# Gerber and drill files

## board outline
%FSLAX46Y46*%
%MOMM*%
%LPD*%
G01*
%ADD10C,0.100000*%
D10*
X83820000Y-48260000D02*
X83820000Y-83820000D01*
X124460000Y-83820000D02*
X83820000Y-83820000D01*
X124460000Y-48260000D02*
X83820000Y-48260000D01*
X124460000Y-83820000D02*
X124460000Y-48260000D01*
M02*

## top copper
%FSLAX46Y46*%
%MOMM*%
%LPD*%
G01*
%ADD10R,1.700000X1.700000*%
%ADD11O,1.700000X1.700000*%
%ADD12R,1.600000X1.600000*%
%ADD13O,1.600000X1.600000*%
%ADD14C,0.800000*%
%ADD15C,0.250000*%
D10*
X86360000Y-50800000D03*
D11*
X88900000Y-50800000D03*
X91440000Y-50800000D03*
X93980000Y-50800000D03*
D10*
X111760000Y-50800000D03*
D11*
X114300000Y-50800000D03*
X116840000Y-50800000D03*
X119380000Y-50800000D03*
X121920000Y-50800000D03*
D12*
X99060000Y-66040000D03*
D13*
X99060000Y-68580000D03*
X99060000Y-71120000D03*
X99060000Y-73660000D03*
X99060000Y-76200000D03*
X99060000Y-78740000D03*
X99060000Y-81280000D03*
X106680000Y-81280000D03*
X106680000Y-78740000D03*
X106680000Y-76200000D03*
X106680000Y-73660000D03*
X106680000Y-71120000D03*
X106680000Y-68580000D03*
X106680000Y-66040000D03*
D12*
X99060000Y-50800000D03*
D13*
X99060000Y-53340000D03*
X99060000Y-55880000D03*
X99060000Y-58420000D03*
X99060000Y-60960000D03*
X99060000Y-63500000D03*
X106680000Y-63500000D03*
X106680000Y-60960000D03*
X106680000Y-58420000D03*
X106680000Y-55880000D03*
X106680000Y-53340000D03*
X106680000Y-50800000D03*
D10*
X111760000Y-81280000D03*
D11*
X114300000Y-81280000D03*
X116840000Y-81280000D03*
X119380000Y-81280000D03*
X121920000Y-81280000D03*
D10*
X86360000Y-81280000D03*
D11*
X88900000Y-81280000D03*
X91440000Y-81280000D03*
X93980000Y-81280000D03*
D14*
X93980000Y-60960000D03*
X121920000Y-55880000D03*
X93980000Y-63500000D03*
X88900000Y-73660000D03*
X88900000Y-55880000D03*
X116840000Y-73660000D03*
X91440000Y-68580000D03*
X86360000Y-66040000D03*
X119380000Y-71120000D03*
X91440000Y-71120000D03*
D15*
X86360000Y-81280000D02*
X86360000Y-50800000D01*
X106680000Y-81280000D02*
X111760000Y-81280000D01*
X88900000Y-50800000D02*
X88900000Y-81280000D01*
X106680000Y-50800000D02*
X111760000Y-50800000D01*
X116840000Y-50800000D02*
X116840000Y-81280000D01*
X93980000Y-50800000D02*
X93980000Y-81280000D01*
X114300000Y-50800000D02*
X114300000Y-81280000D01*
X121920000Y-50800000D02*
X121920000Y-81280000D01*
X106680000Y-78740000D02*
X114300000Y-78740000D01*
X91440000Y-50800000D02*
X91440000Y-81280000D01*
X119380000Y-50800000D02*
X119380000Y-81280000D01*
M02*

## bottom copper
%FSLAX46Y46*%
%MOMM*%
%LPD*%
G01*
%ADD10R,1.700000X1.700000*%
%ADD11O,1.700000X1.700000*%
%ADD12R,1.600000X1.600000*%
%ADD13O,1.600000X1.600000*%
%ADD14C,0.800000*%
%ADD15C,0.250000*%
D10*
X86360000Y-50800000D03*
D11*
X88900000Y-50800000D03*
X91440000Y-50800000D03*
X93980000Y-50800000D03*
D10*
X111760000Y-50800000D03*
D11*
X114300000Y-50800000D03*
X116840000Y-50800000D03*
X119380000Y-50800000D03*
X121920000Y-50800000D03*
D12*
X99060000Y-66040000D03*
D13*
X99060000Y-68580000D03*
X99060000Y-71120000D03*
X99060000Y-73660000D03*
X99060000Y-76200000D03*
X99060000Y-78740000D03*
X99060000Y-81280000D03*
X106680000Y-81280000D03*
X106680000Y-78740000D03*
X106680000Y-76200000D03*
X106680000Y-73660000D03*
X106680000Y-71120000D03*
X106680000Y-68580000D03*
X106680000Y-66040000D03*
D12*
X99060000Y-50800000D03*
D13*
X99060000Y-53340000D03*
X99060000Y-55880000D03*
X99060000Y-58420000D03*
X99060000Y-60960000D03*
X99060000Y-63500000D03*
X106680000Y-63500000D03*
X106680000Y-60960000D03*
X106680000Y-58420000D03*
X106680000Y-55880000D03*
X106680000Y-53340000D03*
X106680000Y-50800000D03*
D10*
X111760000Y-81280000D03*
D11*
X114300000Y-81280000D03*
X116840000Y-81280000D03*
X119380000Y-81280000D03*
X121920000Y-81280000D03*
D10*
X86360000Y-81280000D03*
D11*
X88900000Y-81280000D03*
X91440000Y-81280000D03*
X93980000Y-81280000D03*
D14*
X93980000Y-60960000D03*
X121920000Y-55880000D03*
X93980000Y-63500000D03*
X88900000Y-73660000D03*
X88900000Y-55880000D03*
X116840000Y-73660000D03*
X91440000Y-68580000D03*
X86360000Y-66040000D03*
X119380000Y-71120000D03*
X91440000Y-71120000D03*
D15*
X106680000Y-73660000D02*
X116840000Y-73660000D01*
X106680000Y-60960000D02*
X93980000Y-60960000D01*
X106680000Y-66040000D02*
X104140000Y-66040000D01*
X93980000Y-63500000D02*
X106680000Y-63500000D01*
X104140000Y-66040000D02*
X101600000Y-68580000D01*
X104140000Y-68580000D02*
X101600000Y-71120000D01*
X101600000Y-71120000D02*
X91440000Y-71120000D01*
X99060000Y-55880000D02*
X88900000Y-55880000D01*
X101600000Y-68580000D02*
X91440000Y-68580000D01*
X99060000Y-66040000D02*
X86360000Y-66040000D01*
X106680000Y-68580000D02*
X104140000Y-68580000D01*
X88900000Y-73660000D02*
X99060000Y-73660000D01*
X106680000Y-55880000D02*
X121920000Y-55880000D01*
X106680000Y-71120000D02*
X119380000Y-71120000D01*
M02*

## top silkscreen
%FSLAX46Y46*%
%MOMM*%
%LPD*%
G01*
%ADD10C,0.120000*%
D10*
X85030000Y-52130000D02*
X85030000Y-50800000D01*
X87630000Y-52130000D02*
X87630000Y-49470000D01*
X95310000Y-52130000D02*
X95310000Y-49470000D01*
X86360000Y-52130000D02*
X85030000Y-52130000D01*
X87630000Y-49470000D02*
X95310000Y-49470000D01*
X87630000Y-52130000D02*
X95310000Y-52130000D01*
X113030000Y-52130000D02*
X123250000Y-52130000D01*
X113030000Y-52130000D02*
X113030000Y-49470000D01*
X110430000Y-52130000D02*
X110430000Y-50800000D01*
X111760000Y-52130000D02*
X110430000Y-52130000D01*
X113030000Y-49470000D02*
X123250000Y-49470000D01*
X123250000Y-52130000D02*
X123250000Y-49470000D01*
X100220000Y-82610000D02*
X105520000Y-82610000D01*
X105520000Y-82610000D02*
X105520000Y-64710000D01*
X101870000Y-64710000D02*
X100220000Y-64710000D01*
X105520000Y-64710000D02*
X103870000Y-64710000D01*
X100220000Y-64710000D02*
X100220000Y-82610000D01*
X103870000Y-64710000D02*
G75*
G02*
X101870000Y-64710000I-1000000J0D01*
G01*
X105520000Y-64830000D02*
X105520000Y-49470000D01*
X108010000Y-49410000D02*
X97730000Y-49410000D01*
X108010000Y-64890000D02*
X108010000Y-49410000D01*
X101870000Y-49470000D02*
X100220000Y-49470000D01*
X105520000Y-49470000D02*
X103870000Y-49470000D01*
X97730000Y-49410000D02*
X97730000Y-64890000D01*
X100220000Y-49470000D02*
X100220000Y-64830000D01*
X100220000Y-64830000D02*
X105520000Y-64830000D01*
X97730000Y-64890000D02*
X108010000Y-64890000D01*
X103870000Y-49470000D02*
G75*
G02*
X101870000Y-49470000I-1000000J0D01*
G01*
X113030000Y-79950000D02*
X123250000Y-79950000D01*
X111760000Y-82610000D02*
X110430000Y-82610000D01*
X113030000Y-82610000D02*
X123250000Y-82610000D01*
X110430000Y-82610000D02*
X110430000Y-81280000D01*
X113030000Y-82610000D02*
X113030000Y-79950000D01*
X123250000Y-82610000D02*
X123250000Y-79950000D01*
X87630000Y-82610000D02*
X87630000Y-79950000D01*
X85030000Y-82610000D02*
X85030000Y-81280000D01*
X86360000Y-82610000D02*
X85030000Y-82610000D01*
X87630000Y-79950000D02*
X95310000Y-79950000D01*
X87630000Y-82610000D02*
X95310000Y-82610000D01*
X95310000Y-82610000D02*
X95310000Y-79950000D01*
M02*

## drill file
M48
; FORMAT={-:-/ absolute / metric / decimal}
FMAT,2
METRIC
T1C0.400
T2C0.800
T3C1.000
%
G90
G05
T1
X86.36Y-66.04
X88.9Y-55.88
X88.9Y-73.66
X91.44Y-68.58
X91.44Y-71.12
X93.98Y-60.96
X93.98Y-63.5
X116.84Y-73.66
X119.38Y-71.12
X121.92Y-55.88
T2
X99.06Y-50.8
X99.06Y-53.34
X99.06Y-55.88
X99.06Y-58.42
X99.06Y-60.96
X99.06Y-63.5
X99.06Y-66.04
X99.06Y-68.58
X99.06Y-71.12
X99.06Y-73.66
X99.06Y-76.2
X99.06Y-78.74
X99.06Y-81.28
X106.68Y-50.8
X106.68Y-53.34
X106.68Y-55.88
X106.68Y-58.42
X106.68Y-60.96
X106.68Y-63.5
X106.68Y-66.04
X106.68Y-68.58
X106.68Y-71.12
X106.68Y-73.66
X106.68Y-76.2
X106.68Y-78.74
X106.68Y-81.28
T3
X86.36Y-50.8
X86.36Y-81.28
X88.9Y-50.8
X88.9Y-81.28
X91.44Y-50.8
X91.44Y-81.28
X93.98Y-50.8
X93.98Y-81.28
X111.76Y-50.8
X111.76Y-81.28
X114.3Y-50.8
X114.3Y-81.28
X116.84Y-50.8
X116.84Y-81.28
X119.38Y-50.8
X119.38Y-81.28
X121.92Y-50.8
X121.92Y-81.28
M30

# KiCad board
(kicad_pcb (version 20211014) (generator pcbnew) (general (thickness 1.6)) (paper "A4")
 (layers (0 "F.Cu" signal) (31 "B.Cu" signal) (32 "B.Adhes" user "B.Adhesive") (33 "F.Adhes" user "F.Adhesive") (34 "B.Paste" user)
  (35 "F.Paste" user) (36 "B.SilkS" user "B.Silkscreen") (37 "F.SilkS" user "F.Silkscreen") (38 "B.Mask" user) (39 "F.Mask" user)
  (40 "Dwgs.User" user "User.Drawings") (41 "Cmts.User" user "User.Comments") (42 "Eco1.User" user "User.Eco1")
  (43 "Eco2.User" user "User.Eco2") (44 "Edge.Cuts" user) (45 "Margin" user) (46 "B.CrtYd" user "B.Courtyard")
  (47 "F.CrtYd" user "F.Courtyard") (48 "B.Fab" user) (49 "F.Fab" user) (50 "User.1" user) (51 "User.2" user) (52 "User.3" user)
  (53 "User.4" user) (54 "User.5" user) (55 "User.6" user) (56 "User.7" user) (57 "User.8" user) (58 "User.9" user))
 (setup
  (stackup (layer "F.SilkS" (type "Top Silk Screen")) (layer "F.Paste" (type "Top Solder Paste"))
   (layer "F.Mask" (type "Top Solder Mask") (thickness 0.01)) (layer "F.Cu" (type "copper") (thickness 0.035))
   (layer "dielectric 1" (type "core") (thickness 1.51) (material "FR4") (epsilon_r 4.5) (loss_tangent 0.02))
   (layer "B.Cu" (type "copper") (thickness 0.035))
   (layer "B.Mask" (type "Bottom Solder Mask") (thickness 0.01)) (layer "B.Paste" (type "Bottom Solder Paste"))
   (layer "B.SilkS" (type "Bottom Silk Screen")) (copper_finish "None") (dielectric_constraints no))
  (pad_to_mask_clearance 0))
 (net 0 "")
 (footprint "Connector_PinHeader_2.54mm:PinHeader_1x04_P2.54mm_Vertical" (layer "F.Cu") (at 86.36 50.8 90)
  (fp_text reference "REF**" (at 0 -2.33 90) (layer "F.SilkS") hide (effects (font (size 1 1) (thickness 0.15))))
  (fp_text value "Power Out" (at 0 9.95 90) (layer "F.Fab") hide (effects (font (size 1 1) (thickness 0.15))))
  (fp_line (start -1.33 -1.33) (end 0 -1.33) (layer "F.SilkS") (width 0.12))
  (fp_line (start -1.33 1.27) (end 1.33 1.27) (layer "F.SilkS") (width 0.12))
  (fp_line (start -1.33 8.95) (end 1.33 8.95) (layer "F.SilkS") (width 0.12))
  (fp_line (start -1.33 0) (end -1.33 -1.33) (layer "F.SilkS") (width 0.12))
  (fp_line (start 1.33 1.27) (end 1.33 8.95) (layer "F.SilkS") (width 0.12))
  (fp_line (start -1.33 1.27) (end -1.33 8.95) (layer "F.SilkS") (width 0.12))
  (pad "1" thru_hole rect (at 0 0 90) (size 1.7 1.7) (drill 1) (layers *.Cu *.Mask))
  (pad "2" thru_hole oval (at 0 2.54 90) (size 1.7 1.7) (drill 1) (layers *.Cu *.Mask))
  (pad "3" thru_hole oval (at 0 5.08 90) (size 1.7 1.7) (drill 1) (layers *.Cu *.Mask))
  (pad "4" thru_hole oval (at 0 7.62 90) (size 1.7 1.7) (drill 1) (layers *.Cu *.Mask)))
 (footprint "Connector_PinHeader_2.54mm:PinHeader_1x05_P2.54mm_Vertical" (layer "F.Cu") (at 111.76 50.8 90)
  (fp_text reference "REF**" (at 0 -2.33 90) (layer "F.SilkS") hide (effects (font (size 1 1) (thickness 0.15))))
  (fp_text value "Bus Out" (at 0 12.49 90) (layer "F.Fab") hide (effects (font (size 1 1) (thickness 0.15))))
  (fp_line (start -1.33 1.27) (end -1.33 11.49) (layer "F.SilkS") (width 0.12))
  (fp_line (start -1.33 1.27) (end 1.33 1.27) (layer "F.SilkS") (width 0.12))
  (fp_line (start -1.33 -1.33) (end 0 -1.33) (layer "F.SilkS") (width 0.12))
  (fp_line (start -1.33 0) (end -1.33 -1.33) (layer "F.SilkS") (width 0.12))
  (fp_line (start 1.33 1.27) (end 1.33 11.49) (layer "F.SilkS") (width 0.12))
  (fp_line (start -1.33 11.49) (end 1.33 11.49) (layer "F.SilkS") (width 0.12))
  (pad "1" thru_hole rect (at 0 0 90) (size 1.7 1.7) (drill 1) (layers *.Cu *.Mask))
  (pad "2" thru_hole oval (at 0 2.54 90) (size 1.7 1.7) (drill 1) (layers *.Cu *.Mask))
  (pad "3" thru_hole oval (at 0 5.08 90) (size 1.7 1.7) (drill 1) (layers *.Cu *.Mask))
  (pad "4" thru_hole oval (at 0 7.62 90) (size 1.7 1.7) (drill 1) (layers *.Cu *.Mask))
  (pad "5" thru_hole oval (at 0 10.16 90) (size 1.7 1.7) (drill 1) (layers *.Cu *.Mask)))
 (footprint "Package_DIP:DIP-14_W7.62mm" (layer "F.Cu") (at 99.06 66.04)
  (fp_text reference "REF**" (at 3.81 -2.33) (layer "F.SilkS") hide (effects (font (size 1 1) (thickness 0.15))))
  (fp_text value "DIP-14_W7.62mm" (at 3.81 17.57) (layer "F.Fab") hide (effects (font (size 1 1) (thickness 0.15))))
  (fp_line (start 1.16 16.57) (end 6.46 16.57) (layer "F.SilkS") (width 0.12))
  (fp_line (start 6.46 16.57) (end 6.46 -1.33) (layer "F.SilkS") (width 0.12))
  (fp_line (start 2.81 -1.33) (end 1.16 -1.33) (layer "F.SilkS") (width 0.12))
  (fp_line (start 6.46 -1.33) (end 4.81 -1.33) (layer "F.SilkS") (width 0.12))
  (fp_line (start 1.16 -1.33) (end 1.16 16.57) (layer "F.SilkS") (width 0.12))
  (fp_arc (start 4.81 -1.33) (mid 3.81 -0.33) (end 2.81 -1.33) (layer "F.SilkS") (width 0.12))
  (pad "1" thru_hole rect (at 0 0) (size 1.6 1.6) (drill 0.8) (layers *.Cu *.Mask))
  (pad "2" thru_hole oval (at 0 2.54) (size 1.6 1.6) (drill 0.8) (layers *.Cu *.Mask))
  (pad "3" thru_hole oval (at 0 5.08) (size 1.6 1.6) (drill 0.8) (layers *.Cu *.Mask))
  (pad "4" thru_hole oval (at 0 7.62) (size 1.6 1.6) (drill 0.8) (layers *.Cu *.Mask))
  (pad "5" thru_hole oval (at 0 10.16) (size 1.6 1.6) (drill 0.8) (layers *.Cu *.Mask))
  (pad "6" thru_hole oval (at 0 12.7) (size 1.6 1.6) (drill 0.8) (layers *.Cu *.Mask))
  (pad "7" thru_hole oval (at 0 15.24) (size 1.6 1.6) (drill 0.8) (layers *.Cu *.Mask))
  (pad "8" thru_hole oval (at 7.62 15.24) (size 1.6 1.6) (drill 0.8) (layers *.Cu *.Mask))
  (pad "9" thru_hole oval (at 7.62 12.7) (size 1.6 1.6) (drill 0.8) (layers *.Cu *.Mask))
  (pad "10" thru_hole oval (at 7.62 10.16) (size 1.6 1.6) (drill 0.8) (layers *.Cu *.Mask))
  (pad "11" thru_hole oval (at 7.62 7.62) (size 1.6 1.6) (drill 0.8) (layers *.Cu *.Mask))
  (pad "12" thru_hole oval (at 7.62 5.08) (size 1.6 1.6) (drill 0.8) (layers *.Cu *.Mask))
  (pad "13" thru_hole oval (at 7.62 2.54) (size 1.6 1.6) (drill 0.8) (layers *.Cu *.Mask))
  (pad "14" thru_hole oval (at 7.62 0) (size 1.6 1.6) (drill 0.8) (layers *.Cu *.Mask)))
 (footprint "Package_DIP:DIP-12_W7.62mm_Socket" (layer "F.Cu") (at 99.06 50.8)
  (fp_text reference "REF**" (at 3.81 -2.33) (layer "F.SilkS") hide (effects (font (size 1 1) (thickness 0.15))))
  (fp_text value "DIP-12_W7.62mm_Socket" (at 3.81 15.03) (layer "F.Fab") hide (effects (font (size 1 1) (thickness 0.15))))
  (fp_line (start 6.46 14.03) (end 6.46 -1.33) (layer "F.SilkS") (width 0.12))
  (fp_line (start 8.95 -1.39) (end -1.33 -1.39) (layer "F.SilkS") (width 0.12))
  (fp_line (start 8.95 14.09) (end 8.95 -1.39) (layer "F.SilkS") (width 0.12))
  (fp_line (start 2.81 -1.33) (end 1.16 -1.33) (layer "F.SilkS") (width 0.12))
  (fp_line (start 6.46 -1.33) (end 4.81 -1.33) (layer "F.SilkS") (width 0.12))
  (fp_line (start -1.33 -1.39) (end -1.33 14.09) (layer "F.SilkS") (width 0.12))
  (fp_line (start 1.16 -1.33) (end 1.16 14.03) (layer "F.SilkS") (width 0.12))
  (fp_line (start 1.16 14.03) (end 6.46 14.03) (layer "F.SilkS") (width 0.12))
  (fp_line (start -1.33 14.09) (end 8.95 14.09) (layer "F.SilkS") (width 0.12))
  (fp_arc (start 4.81 -1.33) (mid 3.81 -0.33) (end 2.81 -1.33) (layer "F.SilkS") (width 0.12))
  (pad "1" thru_hole rect (at 0 0) (size 1.6 1.6) (drill 0.8) (layers *.Cu *.Mask))
  (pad "2" thru_hole oval (at 0 2.54) (size 1.6 1.6) (drill 0.8) (layers *.Cu *.Mask))
  (pad "3" thru_hole oval (at 0 5.08) (size 1.6 1.6) (drill 0.8) (layers *.Cu *.Mask))
  (pad "4" thru_hole oval (at 0 7.62) (size 1.6 1.6) (drill 0.8) (layers *.Cu *.Mask))
  (pad "5" thru_hole oval (at 0 10.16) (size 1.6 1.6) (drill 0.8) (layers *.Cu *.Mask))
  (pad "6" thru_hole oval (at 0 12.7) (size 1.6 1.6) (drill 0.8) (layers *.Cu *.Mask))
  (pad "7" thru_hole oval (at 7.62 12.7) (size 1.6 1.6) (drill 0.8) (layers *.Cu *.Mask))
  (pad "8" thru_hole oval (at 7.62 10.16) (size 1.6 1.6) (drill 0.8) (layers *.Cu *.Mask))
  (pad "9" thru_hole oval (at 7.62 7.62) (size 1.6 1.6) (drill 0.8) (layers *.Cu *.Mask))
  (pad "10" thru_hole oval (at 7.62 5.08) (size 1.6 1.6) (drill 0.8) (layers *.Cu *.Mask))
  (pad "11" thru_hole oval (at 7.62 2.54) (size 1.6 1.6) (drill 0.8) (layers *.Cu *.Mask))
  (pad "12" thru_hole oval (at 7.62 0) (size 1.6 1.6) (drill 0.8) (layers *.Cu *.Mask)))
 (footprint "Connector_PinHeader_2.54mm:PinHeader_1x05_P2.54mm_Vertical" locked (layer "F.Cu") (at 111.76 81.28 90)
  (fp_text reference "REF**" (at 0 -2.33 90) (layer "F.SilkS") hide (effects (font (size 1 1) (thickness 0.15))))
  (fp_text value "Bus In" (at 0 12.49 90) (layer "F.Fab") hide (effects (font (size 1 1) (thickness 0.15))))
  (fp_line (start 1.33 1.27) (end 1.33 11.49) (layer "F.SilkS") (width 0.12))
  (fp_line (start -1.33 0) (end -1.33 -1.33) (layer "F.SilkS") (width 0.12))
  (fp_line (start -1.33 1.27) (end -1.33 11.49) (layer "F.SilkS") (width 0.12))
  (fp_line (start -1.33 -1.33) (end 0 -1.33) (layer "F.SilkS") (width 0.12))
  (fp_line (start -1.33 1.27) (end 1.33 1.27) (layer "F.SilkS") (width 0.12))
  (fp_line (start -1.33 11.49) (end 1.33 11.49) (layer "F.SilkS") (width 0.12))
  (pad "1" thru_hole rect locked (at 0 0 90) (size 1.7 1.7) (drill 1) (layers *.Cu *.Mask))
  (pad "2" thru_hole oval locked (at 0 2.54 90) (size 1.7 1.7) (drill 1) (layers *.Cu *.Mask))
  (pad "3" thru_hole oval locked (at 0 5.08 90) (size 1.7 1.7) (drill 1) (layers *.Cu *.Mask))
  (pad "4" thru_hole oval locked (at 0 7.62 90) (size 1.7 1.7) (drill 1) (layers *.Cu *.Mask))
  (pad "5" thru_hole oval locked (at 0 10.16 90) (size 1.7 1.7) (drill 1) (layers *.Cu *.Mask)))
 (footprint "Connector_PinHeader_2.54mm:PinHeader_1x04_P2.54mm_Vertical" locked (layer "F.Cu") (at 86.36 81.28 90)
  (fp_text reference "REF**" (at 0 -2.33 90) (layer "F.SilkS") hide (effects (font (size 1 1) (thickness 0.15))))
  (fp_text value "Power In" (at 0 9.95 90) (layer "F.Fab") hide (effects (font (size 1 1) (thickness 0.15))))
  (fp_line (start -1.33 1.27) (end 1.33 1.27) (layer "F.SilkS") (width 0.12))
  (fp_line (start -1.33 -1.33) (end 0 -1.33) (layer "F.SilkS") (width 0.12))
  (fp_line (start -1.33 0) (end -1.33 -1.33) (layer "F.SilkS") (width 0.12))
  (fp_line (start 1.33 1.27) (end 1.33 8.95) (layer "F.SilkS") (width 0.12))
  (fp_line (start -1.33 1.27) (end -1.33 8.95) (layer "F.SilkS") (width 0.12))
  (fp_line (start -1.33 8.95) (end 1.33 8.95) (layer "F.SilkS") (width 0.12))
  (pad "1" thru_hole rect locked (at 0 0 90) (size 1.7 1.7) (drill 1) (layers *.Cu *.Mask))
  (pad "2" thru_hole oval locked (at 0 2.54 90) (size 1.7 1.7) (drill 1) (layers *.Cu *.Mask))
  (pad "3" thru_hole oval locked (at 0 5.08 90) (size 1.7 1.7) (drill 1) (layers *.Cu *.Mask))
  (pad "4" thru_hole oval locked (at 0 7.62 90) (size 1.7 1.7) (drill 1) (layers *.Cu *.Mask)))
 (gr_line (start 83.82 48.26) (end 83.82 83.82) (layer "Edge.Cuts") (width 0.1))
 (gr_line (start 124.46 83.82) (end 83.82 83.82) (layer "Edge.Cuts") (width 0.1))
 (gr_line (start 124.46 48.26) (end 83.82 48.26) (layer "Edge.Cuts") (width 0.1))
 (gr_line (start 124.46 83.82) (end 124.46 48.26) (layer "Edge.Cuts") (width 0.1))
 (segment (start 86.36 81.28) (end 86.36 50.8) (width 0.25) (layer "F.Cu") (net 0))
 (segment (start 106.68 81.28) (end 111.76 81.28) (width 0.25) (layer "F.Cu") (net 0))
 (segment (start 88.9 50.8) (end 88.9 81.28) (width 0.25) (layer "F.Cu") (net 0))
 (segment (start 106.68 50.8) (end 111.76 50.8) (width 0.25) (layer "F.Cu") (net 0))
 (segment (start 116.84 50.8) (end 116.84 81.28) (width 0.25) (layer "F.Cu") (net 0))
 (segment (start 93.98 50.8) (end 93.98 81.28) (width 0.25) (layer "F.Cu") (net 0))
 (segment (start 114.3 50.8) (end 114.3 81.28) (width 0.25) (layer "F.Cu") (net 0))
 (segment (start 121.92 50.8) (end 121.92 81.28) (width 0.25) (layer "F.Cu") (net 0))
 (segment (start 106.68 78.74) (end 114.3 78.74) (width 0.25) (layer "F.Cu") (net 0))
 (segment (start 91.44 50.8) (end 91.44 81.28) (width 0.25) (layer "F.Cu") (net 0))
 (segment (start 119.38 50.8) (end 119.38 81.28) (width 0.25) (layer "F.Cu") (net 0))
 (via (at 93.98 60.96) (size 0.8) (drill 0.4) (layers "F.Cu" "B.Cu") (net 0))
 (via (at 121.92 55.88) (size 0.8) (drill 0.4) (layers "F.Cu" "B.Cu") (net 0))
 (via (at 93.98 63.5) (size 0.8) (drill 0.4) (layers "F.Cu" "B.Cu") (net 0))
 (via (at 88.9 73.66) (size 0.8) (drill 0.4) (layers "F.Cu" "B.Cu") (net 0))
 (via (at 88.9 55.88) (size 0.8) (drill 0.4) (layers "F.Cu" "B.Cu") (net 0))
 (via (at 116.84 73.66) (size 0.8) (drill 0.4) (layers "F.Cu" "B.Cu") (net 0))
 (via (at 91.44 68.58) (size 0.8) (drill 0.4) (layers "F.Cu" "B.Cu") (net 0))
 (via (at 86.36 66.04) (size 0.8) (drill 0.4) (layers "F.Cu" "B.Cu") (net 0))
 (via (at 119.38 71.12) (size 0.8) (drill 0.4) (layers "F.Cu" "B.Cu") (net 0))
 (via (at 91.44 71.12) (size 0.8) (drill 0.4) (layers "F.Cu" "B.Cu") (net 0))
 (segment (start 106.68 73.66) (end 116.84 73.66) (width 0.25) (layer "B.Cu") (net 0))
 (segment (start 106.68 60.96) (end 93.98 60.96) (width 0.25) (layer "B.Cu") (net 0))
 (segment (start 106.68 66.04) (end 104.14 66.04) (width 0.25) (layer "B.Cu") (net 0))
 (segment (start 93.98 63.5) (end 106.68 63.5) (width 0.25) (layer "B.Cu") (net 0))
 (segment (start 104.14 66.04) (end 101.6 68.58) (width 0.25) (layer "B.Cu") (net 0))
 (segment (start 104.14 68.58) (end 101.6 71.12) (width 0.25) (layer "B.Cu") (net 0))
 (segment (start 101.6 71.12) (end 91.44 71.12) (width 0.25) (layer "B.Cu") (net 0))
 (segment (start 99.06 55.88) (end 88.9 55.88) (width 0.25) (layer "B.Cu") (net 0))
 (segment (start 101.6 68.58) (end 91.44 68.58) (width 0.25) (layer "B.Cu") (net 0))
 (segment (start 99.06 66.04) (end 86.36 66.04) (width 0.25) (layer "B.Cu") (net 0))
 (segment (start 106.68 68.58) (end 104.14 68.58) (width 0.25) (layer "B.Cu") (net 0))
 (segment (start 88.9 73.66) (end 99.06 73.66) (width 0.25) (layer "B.Cu") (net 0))
 (segment (start 106.68 55.88) (end 121.92 55.88) (width 0.25) (layer "B.Cu") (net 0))
 (segment (start 106.68 71.12) (end 119.38 71.12) (width 0.25) (layer "B.Cu") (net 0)))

